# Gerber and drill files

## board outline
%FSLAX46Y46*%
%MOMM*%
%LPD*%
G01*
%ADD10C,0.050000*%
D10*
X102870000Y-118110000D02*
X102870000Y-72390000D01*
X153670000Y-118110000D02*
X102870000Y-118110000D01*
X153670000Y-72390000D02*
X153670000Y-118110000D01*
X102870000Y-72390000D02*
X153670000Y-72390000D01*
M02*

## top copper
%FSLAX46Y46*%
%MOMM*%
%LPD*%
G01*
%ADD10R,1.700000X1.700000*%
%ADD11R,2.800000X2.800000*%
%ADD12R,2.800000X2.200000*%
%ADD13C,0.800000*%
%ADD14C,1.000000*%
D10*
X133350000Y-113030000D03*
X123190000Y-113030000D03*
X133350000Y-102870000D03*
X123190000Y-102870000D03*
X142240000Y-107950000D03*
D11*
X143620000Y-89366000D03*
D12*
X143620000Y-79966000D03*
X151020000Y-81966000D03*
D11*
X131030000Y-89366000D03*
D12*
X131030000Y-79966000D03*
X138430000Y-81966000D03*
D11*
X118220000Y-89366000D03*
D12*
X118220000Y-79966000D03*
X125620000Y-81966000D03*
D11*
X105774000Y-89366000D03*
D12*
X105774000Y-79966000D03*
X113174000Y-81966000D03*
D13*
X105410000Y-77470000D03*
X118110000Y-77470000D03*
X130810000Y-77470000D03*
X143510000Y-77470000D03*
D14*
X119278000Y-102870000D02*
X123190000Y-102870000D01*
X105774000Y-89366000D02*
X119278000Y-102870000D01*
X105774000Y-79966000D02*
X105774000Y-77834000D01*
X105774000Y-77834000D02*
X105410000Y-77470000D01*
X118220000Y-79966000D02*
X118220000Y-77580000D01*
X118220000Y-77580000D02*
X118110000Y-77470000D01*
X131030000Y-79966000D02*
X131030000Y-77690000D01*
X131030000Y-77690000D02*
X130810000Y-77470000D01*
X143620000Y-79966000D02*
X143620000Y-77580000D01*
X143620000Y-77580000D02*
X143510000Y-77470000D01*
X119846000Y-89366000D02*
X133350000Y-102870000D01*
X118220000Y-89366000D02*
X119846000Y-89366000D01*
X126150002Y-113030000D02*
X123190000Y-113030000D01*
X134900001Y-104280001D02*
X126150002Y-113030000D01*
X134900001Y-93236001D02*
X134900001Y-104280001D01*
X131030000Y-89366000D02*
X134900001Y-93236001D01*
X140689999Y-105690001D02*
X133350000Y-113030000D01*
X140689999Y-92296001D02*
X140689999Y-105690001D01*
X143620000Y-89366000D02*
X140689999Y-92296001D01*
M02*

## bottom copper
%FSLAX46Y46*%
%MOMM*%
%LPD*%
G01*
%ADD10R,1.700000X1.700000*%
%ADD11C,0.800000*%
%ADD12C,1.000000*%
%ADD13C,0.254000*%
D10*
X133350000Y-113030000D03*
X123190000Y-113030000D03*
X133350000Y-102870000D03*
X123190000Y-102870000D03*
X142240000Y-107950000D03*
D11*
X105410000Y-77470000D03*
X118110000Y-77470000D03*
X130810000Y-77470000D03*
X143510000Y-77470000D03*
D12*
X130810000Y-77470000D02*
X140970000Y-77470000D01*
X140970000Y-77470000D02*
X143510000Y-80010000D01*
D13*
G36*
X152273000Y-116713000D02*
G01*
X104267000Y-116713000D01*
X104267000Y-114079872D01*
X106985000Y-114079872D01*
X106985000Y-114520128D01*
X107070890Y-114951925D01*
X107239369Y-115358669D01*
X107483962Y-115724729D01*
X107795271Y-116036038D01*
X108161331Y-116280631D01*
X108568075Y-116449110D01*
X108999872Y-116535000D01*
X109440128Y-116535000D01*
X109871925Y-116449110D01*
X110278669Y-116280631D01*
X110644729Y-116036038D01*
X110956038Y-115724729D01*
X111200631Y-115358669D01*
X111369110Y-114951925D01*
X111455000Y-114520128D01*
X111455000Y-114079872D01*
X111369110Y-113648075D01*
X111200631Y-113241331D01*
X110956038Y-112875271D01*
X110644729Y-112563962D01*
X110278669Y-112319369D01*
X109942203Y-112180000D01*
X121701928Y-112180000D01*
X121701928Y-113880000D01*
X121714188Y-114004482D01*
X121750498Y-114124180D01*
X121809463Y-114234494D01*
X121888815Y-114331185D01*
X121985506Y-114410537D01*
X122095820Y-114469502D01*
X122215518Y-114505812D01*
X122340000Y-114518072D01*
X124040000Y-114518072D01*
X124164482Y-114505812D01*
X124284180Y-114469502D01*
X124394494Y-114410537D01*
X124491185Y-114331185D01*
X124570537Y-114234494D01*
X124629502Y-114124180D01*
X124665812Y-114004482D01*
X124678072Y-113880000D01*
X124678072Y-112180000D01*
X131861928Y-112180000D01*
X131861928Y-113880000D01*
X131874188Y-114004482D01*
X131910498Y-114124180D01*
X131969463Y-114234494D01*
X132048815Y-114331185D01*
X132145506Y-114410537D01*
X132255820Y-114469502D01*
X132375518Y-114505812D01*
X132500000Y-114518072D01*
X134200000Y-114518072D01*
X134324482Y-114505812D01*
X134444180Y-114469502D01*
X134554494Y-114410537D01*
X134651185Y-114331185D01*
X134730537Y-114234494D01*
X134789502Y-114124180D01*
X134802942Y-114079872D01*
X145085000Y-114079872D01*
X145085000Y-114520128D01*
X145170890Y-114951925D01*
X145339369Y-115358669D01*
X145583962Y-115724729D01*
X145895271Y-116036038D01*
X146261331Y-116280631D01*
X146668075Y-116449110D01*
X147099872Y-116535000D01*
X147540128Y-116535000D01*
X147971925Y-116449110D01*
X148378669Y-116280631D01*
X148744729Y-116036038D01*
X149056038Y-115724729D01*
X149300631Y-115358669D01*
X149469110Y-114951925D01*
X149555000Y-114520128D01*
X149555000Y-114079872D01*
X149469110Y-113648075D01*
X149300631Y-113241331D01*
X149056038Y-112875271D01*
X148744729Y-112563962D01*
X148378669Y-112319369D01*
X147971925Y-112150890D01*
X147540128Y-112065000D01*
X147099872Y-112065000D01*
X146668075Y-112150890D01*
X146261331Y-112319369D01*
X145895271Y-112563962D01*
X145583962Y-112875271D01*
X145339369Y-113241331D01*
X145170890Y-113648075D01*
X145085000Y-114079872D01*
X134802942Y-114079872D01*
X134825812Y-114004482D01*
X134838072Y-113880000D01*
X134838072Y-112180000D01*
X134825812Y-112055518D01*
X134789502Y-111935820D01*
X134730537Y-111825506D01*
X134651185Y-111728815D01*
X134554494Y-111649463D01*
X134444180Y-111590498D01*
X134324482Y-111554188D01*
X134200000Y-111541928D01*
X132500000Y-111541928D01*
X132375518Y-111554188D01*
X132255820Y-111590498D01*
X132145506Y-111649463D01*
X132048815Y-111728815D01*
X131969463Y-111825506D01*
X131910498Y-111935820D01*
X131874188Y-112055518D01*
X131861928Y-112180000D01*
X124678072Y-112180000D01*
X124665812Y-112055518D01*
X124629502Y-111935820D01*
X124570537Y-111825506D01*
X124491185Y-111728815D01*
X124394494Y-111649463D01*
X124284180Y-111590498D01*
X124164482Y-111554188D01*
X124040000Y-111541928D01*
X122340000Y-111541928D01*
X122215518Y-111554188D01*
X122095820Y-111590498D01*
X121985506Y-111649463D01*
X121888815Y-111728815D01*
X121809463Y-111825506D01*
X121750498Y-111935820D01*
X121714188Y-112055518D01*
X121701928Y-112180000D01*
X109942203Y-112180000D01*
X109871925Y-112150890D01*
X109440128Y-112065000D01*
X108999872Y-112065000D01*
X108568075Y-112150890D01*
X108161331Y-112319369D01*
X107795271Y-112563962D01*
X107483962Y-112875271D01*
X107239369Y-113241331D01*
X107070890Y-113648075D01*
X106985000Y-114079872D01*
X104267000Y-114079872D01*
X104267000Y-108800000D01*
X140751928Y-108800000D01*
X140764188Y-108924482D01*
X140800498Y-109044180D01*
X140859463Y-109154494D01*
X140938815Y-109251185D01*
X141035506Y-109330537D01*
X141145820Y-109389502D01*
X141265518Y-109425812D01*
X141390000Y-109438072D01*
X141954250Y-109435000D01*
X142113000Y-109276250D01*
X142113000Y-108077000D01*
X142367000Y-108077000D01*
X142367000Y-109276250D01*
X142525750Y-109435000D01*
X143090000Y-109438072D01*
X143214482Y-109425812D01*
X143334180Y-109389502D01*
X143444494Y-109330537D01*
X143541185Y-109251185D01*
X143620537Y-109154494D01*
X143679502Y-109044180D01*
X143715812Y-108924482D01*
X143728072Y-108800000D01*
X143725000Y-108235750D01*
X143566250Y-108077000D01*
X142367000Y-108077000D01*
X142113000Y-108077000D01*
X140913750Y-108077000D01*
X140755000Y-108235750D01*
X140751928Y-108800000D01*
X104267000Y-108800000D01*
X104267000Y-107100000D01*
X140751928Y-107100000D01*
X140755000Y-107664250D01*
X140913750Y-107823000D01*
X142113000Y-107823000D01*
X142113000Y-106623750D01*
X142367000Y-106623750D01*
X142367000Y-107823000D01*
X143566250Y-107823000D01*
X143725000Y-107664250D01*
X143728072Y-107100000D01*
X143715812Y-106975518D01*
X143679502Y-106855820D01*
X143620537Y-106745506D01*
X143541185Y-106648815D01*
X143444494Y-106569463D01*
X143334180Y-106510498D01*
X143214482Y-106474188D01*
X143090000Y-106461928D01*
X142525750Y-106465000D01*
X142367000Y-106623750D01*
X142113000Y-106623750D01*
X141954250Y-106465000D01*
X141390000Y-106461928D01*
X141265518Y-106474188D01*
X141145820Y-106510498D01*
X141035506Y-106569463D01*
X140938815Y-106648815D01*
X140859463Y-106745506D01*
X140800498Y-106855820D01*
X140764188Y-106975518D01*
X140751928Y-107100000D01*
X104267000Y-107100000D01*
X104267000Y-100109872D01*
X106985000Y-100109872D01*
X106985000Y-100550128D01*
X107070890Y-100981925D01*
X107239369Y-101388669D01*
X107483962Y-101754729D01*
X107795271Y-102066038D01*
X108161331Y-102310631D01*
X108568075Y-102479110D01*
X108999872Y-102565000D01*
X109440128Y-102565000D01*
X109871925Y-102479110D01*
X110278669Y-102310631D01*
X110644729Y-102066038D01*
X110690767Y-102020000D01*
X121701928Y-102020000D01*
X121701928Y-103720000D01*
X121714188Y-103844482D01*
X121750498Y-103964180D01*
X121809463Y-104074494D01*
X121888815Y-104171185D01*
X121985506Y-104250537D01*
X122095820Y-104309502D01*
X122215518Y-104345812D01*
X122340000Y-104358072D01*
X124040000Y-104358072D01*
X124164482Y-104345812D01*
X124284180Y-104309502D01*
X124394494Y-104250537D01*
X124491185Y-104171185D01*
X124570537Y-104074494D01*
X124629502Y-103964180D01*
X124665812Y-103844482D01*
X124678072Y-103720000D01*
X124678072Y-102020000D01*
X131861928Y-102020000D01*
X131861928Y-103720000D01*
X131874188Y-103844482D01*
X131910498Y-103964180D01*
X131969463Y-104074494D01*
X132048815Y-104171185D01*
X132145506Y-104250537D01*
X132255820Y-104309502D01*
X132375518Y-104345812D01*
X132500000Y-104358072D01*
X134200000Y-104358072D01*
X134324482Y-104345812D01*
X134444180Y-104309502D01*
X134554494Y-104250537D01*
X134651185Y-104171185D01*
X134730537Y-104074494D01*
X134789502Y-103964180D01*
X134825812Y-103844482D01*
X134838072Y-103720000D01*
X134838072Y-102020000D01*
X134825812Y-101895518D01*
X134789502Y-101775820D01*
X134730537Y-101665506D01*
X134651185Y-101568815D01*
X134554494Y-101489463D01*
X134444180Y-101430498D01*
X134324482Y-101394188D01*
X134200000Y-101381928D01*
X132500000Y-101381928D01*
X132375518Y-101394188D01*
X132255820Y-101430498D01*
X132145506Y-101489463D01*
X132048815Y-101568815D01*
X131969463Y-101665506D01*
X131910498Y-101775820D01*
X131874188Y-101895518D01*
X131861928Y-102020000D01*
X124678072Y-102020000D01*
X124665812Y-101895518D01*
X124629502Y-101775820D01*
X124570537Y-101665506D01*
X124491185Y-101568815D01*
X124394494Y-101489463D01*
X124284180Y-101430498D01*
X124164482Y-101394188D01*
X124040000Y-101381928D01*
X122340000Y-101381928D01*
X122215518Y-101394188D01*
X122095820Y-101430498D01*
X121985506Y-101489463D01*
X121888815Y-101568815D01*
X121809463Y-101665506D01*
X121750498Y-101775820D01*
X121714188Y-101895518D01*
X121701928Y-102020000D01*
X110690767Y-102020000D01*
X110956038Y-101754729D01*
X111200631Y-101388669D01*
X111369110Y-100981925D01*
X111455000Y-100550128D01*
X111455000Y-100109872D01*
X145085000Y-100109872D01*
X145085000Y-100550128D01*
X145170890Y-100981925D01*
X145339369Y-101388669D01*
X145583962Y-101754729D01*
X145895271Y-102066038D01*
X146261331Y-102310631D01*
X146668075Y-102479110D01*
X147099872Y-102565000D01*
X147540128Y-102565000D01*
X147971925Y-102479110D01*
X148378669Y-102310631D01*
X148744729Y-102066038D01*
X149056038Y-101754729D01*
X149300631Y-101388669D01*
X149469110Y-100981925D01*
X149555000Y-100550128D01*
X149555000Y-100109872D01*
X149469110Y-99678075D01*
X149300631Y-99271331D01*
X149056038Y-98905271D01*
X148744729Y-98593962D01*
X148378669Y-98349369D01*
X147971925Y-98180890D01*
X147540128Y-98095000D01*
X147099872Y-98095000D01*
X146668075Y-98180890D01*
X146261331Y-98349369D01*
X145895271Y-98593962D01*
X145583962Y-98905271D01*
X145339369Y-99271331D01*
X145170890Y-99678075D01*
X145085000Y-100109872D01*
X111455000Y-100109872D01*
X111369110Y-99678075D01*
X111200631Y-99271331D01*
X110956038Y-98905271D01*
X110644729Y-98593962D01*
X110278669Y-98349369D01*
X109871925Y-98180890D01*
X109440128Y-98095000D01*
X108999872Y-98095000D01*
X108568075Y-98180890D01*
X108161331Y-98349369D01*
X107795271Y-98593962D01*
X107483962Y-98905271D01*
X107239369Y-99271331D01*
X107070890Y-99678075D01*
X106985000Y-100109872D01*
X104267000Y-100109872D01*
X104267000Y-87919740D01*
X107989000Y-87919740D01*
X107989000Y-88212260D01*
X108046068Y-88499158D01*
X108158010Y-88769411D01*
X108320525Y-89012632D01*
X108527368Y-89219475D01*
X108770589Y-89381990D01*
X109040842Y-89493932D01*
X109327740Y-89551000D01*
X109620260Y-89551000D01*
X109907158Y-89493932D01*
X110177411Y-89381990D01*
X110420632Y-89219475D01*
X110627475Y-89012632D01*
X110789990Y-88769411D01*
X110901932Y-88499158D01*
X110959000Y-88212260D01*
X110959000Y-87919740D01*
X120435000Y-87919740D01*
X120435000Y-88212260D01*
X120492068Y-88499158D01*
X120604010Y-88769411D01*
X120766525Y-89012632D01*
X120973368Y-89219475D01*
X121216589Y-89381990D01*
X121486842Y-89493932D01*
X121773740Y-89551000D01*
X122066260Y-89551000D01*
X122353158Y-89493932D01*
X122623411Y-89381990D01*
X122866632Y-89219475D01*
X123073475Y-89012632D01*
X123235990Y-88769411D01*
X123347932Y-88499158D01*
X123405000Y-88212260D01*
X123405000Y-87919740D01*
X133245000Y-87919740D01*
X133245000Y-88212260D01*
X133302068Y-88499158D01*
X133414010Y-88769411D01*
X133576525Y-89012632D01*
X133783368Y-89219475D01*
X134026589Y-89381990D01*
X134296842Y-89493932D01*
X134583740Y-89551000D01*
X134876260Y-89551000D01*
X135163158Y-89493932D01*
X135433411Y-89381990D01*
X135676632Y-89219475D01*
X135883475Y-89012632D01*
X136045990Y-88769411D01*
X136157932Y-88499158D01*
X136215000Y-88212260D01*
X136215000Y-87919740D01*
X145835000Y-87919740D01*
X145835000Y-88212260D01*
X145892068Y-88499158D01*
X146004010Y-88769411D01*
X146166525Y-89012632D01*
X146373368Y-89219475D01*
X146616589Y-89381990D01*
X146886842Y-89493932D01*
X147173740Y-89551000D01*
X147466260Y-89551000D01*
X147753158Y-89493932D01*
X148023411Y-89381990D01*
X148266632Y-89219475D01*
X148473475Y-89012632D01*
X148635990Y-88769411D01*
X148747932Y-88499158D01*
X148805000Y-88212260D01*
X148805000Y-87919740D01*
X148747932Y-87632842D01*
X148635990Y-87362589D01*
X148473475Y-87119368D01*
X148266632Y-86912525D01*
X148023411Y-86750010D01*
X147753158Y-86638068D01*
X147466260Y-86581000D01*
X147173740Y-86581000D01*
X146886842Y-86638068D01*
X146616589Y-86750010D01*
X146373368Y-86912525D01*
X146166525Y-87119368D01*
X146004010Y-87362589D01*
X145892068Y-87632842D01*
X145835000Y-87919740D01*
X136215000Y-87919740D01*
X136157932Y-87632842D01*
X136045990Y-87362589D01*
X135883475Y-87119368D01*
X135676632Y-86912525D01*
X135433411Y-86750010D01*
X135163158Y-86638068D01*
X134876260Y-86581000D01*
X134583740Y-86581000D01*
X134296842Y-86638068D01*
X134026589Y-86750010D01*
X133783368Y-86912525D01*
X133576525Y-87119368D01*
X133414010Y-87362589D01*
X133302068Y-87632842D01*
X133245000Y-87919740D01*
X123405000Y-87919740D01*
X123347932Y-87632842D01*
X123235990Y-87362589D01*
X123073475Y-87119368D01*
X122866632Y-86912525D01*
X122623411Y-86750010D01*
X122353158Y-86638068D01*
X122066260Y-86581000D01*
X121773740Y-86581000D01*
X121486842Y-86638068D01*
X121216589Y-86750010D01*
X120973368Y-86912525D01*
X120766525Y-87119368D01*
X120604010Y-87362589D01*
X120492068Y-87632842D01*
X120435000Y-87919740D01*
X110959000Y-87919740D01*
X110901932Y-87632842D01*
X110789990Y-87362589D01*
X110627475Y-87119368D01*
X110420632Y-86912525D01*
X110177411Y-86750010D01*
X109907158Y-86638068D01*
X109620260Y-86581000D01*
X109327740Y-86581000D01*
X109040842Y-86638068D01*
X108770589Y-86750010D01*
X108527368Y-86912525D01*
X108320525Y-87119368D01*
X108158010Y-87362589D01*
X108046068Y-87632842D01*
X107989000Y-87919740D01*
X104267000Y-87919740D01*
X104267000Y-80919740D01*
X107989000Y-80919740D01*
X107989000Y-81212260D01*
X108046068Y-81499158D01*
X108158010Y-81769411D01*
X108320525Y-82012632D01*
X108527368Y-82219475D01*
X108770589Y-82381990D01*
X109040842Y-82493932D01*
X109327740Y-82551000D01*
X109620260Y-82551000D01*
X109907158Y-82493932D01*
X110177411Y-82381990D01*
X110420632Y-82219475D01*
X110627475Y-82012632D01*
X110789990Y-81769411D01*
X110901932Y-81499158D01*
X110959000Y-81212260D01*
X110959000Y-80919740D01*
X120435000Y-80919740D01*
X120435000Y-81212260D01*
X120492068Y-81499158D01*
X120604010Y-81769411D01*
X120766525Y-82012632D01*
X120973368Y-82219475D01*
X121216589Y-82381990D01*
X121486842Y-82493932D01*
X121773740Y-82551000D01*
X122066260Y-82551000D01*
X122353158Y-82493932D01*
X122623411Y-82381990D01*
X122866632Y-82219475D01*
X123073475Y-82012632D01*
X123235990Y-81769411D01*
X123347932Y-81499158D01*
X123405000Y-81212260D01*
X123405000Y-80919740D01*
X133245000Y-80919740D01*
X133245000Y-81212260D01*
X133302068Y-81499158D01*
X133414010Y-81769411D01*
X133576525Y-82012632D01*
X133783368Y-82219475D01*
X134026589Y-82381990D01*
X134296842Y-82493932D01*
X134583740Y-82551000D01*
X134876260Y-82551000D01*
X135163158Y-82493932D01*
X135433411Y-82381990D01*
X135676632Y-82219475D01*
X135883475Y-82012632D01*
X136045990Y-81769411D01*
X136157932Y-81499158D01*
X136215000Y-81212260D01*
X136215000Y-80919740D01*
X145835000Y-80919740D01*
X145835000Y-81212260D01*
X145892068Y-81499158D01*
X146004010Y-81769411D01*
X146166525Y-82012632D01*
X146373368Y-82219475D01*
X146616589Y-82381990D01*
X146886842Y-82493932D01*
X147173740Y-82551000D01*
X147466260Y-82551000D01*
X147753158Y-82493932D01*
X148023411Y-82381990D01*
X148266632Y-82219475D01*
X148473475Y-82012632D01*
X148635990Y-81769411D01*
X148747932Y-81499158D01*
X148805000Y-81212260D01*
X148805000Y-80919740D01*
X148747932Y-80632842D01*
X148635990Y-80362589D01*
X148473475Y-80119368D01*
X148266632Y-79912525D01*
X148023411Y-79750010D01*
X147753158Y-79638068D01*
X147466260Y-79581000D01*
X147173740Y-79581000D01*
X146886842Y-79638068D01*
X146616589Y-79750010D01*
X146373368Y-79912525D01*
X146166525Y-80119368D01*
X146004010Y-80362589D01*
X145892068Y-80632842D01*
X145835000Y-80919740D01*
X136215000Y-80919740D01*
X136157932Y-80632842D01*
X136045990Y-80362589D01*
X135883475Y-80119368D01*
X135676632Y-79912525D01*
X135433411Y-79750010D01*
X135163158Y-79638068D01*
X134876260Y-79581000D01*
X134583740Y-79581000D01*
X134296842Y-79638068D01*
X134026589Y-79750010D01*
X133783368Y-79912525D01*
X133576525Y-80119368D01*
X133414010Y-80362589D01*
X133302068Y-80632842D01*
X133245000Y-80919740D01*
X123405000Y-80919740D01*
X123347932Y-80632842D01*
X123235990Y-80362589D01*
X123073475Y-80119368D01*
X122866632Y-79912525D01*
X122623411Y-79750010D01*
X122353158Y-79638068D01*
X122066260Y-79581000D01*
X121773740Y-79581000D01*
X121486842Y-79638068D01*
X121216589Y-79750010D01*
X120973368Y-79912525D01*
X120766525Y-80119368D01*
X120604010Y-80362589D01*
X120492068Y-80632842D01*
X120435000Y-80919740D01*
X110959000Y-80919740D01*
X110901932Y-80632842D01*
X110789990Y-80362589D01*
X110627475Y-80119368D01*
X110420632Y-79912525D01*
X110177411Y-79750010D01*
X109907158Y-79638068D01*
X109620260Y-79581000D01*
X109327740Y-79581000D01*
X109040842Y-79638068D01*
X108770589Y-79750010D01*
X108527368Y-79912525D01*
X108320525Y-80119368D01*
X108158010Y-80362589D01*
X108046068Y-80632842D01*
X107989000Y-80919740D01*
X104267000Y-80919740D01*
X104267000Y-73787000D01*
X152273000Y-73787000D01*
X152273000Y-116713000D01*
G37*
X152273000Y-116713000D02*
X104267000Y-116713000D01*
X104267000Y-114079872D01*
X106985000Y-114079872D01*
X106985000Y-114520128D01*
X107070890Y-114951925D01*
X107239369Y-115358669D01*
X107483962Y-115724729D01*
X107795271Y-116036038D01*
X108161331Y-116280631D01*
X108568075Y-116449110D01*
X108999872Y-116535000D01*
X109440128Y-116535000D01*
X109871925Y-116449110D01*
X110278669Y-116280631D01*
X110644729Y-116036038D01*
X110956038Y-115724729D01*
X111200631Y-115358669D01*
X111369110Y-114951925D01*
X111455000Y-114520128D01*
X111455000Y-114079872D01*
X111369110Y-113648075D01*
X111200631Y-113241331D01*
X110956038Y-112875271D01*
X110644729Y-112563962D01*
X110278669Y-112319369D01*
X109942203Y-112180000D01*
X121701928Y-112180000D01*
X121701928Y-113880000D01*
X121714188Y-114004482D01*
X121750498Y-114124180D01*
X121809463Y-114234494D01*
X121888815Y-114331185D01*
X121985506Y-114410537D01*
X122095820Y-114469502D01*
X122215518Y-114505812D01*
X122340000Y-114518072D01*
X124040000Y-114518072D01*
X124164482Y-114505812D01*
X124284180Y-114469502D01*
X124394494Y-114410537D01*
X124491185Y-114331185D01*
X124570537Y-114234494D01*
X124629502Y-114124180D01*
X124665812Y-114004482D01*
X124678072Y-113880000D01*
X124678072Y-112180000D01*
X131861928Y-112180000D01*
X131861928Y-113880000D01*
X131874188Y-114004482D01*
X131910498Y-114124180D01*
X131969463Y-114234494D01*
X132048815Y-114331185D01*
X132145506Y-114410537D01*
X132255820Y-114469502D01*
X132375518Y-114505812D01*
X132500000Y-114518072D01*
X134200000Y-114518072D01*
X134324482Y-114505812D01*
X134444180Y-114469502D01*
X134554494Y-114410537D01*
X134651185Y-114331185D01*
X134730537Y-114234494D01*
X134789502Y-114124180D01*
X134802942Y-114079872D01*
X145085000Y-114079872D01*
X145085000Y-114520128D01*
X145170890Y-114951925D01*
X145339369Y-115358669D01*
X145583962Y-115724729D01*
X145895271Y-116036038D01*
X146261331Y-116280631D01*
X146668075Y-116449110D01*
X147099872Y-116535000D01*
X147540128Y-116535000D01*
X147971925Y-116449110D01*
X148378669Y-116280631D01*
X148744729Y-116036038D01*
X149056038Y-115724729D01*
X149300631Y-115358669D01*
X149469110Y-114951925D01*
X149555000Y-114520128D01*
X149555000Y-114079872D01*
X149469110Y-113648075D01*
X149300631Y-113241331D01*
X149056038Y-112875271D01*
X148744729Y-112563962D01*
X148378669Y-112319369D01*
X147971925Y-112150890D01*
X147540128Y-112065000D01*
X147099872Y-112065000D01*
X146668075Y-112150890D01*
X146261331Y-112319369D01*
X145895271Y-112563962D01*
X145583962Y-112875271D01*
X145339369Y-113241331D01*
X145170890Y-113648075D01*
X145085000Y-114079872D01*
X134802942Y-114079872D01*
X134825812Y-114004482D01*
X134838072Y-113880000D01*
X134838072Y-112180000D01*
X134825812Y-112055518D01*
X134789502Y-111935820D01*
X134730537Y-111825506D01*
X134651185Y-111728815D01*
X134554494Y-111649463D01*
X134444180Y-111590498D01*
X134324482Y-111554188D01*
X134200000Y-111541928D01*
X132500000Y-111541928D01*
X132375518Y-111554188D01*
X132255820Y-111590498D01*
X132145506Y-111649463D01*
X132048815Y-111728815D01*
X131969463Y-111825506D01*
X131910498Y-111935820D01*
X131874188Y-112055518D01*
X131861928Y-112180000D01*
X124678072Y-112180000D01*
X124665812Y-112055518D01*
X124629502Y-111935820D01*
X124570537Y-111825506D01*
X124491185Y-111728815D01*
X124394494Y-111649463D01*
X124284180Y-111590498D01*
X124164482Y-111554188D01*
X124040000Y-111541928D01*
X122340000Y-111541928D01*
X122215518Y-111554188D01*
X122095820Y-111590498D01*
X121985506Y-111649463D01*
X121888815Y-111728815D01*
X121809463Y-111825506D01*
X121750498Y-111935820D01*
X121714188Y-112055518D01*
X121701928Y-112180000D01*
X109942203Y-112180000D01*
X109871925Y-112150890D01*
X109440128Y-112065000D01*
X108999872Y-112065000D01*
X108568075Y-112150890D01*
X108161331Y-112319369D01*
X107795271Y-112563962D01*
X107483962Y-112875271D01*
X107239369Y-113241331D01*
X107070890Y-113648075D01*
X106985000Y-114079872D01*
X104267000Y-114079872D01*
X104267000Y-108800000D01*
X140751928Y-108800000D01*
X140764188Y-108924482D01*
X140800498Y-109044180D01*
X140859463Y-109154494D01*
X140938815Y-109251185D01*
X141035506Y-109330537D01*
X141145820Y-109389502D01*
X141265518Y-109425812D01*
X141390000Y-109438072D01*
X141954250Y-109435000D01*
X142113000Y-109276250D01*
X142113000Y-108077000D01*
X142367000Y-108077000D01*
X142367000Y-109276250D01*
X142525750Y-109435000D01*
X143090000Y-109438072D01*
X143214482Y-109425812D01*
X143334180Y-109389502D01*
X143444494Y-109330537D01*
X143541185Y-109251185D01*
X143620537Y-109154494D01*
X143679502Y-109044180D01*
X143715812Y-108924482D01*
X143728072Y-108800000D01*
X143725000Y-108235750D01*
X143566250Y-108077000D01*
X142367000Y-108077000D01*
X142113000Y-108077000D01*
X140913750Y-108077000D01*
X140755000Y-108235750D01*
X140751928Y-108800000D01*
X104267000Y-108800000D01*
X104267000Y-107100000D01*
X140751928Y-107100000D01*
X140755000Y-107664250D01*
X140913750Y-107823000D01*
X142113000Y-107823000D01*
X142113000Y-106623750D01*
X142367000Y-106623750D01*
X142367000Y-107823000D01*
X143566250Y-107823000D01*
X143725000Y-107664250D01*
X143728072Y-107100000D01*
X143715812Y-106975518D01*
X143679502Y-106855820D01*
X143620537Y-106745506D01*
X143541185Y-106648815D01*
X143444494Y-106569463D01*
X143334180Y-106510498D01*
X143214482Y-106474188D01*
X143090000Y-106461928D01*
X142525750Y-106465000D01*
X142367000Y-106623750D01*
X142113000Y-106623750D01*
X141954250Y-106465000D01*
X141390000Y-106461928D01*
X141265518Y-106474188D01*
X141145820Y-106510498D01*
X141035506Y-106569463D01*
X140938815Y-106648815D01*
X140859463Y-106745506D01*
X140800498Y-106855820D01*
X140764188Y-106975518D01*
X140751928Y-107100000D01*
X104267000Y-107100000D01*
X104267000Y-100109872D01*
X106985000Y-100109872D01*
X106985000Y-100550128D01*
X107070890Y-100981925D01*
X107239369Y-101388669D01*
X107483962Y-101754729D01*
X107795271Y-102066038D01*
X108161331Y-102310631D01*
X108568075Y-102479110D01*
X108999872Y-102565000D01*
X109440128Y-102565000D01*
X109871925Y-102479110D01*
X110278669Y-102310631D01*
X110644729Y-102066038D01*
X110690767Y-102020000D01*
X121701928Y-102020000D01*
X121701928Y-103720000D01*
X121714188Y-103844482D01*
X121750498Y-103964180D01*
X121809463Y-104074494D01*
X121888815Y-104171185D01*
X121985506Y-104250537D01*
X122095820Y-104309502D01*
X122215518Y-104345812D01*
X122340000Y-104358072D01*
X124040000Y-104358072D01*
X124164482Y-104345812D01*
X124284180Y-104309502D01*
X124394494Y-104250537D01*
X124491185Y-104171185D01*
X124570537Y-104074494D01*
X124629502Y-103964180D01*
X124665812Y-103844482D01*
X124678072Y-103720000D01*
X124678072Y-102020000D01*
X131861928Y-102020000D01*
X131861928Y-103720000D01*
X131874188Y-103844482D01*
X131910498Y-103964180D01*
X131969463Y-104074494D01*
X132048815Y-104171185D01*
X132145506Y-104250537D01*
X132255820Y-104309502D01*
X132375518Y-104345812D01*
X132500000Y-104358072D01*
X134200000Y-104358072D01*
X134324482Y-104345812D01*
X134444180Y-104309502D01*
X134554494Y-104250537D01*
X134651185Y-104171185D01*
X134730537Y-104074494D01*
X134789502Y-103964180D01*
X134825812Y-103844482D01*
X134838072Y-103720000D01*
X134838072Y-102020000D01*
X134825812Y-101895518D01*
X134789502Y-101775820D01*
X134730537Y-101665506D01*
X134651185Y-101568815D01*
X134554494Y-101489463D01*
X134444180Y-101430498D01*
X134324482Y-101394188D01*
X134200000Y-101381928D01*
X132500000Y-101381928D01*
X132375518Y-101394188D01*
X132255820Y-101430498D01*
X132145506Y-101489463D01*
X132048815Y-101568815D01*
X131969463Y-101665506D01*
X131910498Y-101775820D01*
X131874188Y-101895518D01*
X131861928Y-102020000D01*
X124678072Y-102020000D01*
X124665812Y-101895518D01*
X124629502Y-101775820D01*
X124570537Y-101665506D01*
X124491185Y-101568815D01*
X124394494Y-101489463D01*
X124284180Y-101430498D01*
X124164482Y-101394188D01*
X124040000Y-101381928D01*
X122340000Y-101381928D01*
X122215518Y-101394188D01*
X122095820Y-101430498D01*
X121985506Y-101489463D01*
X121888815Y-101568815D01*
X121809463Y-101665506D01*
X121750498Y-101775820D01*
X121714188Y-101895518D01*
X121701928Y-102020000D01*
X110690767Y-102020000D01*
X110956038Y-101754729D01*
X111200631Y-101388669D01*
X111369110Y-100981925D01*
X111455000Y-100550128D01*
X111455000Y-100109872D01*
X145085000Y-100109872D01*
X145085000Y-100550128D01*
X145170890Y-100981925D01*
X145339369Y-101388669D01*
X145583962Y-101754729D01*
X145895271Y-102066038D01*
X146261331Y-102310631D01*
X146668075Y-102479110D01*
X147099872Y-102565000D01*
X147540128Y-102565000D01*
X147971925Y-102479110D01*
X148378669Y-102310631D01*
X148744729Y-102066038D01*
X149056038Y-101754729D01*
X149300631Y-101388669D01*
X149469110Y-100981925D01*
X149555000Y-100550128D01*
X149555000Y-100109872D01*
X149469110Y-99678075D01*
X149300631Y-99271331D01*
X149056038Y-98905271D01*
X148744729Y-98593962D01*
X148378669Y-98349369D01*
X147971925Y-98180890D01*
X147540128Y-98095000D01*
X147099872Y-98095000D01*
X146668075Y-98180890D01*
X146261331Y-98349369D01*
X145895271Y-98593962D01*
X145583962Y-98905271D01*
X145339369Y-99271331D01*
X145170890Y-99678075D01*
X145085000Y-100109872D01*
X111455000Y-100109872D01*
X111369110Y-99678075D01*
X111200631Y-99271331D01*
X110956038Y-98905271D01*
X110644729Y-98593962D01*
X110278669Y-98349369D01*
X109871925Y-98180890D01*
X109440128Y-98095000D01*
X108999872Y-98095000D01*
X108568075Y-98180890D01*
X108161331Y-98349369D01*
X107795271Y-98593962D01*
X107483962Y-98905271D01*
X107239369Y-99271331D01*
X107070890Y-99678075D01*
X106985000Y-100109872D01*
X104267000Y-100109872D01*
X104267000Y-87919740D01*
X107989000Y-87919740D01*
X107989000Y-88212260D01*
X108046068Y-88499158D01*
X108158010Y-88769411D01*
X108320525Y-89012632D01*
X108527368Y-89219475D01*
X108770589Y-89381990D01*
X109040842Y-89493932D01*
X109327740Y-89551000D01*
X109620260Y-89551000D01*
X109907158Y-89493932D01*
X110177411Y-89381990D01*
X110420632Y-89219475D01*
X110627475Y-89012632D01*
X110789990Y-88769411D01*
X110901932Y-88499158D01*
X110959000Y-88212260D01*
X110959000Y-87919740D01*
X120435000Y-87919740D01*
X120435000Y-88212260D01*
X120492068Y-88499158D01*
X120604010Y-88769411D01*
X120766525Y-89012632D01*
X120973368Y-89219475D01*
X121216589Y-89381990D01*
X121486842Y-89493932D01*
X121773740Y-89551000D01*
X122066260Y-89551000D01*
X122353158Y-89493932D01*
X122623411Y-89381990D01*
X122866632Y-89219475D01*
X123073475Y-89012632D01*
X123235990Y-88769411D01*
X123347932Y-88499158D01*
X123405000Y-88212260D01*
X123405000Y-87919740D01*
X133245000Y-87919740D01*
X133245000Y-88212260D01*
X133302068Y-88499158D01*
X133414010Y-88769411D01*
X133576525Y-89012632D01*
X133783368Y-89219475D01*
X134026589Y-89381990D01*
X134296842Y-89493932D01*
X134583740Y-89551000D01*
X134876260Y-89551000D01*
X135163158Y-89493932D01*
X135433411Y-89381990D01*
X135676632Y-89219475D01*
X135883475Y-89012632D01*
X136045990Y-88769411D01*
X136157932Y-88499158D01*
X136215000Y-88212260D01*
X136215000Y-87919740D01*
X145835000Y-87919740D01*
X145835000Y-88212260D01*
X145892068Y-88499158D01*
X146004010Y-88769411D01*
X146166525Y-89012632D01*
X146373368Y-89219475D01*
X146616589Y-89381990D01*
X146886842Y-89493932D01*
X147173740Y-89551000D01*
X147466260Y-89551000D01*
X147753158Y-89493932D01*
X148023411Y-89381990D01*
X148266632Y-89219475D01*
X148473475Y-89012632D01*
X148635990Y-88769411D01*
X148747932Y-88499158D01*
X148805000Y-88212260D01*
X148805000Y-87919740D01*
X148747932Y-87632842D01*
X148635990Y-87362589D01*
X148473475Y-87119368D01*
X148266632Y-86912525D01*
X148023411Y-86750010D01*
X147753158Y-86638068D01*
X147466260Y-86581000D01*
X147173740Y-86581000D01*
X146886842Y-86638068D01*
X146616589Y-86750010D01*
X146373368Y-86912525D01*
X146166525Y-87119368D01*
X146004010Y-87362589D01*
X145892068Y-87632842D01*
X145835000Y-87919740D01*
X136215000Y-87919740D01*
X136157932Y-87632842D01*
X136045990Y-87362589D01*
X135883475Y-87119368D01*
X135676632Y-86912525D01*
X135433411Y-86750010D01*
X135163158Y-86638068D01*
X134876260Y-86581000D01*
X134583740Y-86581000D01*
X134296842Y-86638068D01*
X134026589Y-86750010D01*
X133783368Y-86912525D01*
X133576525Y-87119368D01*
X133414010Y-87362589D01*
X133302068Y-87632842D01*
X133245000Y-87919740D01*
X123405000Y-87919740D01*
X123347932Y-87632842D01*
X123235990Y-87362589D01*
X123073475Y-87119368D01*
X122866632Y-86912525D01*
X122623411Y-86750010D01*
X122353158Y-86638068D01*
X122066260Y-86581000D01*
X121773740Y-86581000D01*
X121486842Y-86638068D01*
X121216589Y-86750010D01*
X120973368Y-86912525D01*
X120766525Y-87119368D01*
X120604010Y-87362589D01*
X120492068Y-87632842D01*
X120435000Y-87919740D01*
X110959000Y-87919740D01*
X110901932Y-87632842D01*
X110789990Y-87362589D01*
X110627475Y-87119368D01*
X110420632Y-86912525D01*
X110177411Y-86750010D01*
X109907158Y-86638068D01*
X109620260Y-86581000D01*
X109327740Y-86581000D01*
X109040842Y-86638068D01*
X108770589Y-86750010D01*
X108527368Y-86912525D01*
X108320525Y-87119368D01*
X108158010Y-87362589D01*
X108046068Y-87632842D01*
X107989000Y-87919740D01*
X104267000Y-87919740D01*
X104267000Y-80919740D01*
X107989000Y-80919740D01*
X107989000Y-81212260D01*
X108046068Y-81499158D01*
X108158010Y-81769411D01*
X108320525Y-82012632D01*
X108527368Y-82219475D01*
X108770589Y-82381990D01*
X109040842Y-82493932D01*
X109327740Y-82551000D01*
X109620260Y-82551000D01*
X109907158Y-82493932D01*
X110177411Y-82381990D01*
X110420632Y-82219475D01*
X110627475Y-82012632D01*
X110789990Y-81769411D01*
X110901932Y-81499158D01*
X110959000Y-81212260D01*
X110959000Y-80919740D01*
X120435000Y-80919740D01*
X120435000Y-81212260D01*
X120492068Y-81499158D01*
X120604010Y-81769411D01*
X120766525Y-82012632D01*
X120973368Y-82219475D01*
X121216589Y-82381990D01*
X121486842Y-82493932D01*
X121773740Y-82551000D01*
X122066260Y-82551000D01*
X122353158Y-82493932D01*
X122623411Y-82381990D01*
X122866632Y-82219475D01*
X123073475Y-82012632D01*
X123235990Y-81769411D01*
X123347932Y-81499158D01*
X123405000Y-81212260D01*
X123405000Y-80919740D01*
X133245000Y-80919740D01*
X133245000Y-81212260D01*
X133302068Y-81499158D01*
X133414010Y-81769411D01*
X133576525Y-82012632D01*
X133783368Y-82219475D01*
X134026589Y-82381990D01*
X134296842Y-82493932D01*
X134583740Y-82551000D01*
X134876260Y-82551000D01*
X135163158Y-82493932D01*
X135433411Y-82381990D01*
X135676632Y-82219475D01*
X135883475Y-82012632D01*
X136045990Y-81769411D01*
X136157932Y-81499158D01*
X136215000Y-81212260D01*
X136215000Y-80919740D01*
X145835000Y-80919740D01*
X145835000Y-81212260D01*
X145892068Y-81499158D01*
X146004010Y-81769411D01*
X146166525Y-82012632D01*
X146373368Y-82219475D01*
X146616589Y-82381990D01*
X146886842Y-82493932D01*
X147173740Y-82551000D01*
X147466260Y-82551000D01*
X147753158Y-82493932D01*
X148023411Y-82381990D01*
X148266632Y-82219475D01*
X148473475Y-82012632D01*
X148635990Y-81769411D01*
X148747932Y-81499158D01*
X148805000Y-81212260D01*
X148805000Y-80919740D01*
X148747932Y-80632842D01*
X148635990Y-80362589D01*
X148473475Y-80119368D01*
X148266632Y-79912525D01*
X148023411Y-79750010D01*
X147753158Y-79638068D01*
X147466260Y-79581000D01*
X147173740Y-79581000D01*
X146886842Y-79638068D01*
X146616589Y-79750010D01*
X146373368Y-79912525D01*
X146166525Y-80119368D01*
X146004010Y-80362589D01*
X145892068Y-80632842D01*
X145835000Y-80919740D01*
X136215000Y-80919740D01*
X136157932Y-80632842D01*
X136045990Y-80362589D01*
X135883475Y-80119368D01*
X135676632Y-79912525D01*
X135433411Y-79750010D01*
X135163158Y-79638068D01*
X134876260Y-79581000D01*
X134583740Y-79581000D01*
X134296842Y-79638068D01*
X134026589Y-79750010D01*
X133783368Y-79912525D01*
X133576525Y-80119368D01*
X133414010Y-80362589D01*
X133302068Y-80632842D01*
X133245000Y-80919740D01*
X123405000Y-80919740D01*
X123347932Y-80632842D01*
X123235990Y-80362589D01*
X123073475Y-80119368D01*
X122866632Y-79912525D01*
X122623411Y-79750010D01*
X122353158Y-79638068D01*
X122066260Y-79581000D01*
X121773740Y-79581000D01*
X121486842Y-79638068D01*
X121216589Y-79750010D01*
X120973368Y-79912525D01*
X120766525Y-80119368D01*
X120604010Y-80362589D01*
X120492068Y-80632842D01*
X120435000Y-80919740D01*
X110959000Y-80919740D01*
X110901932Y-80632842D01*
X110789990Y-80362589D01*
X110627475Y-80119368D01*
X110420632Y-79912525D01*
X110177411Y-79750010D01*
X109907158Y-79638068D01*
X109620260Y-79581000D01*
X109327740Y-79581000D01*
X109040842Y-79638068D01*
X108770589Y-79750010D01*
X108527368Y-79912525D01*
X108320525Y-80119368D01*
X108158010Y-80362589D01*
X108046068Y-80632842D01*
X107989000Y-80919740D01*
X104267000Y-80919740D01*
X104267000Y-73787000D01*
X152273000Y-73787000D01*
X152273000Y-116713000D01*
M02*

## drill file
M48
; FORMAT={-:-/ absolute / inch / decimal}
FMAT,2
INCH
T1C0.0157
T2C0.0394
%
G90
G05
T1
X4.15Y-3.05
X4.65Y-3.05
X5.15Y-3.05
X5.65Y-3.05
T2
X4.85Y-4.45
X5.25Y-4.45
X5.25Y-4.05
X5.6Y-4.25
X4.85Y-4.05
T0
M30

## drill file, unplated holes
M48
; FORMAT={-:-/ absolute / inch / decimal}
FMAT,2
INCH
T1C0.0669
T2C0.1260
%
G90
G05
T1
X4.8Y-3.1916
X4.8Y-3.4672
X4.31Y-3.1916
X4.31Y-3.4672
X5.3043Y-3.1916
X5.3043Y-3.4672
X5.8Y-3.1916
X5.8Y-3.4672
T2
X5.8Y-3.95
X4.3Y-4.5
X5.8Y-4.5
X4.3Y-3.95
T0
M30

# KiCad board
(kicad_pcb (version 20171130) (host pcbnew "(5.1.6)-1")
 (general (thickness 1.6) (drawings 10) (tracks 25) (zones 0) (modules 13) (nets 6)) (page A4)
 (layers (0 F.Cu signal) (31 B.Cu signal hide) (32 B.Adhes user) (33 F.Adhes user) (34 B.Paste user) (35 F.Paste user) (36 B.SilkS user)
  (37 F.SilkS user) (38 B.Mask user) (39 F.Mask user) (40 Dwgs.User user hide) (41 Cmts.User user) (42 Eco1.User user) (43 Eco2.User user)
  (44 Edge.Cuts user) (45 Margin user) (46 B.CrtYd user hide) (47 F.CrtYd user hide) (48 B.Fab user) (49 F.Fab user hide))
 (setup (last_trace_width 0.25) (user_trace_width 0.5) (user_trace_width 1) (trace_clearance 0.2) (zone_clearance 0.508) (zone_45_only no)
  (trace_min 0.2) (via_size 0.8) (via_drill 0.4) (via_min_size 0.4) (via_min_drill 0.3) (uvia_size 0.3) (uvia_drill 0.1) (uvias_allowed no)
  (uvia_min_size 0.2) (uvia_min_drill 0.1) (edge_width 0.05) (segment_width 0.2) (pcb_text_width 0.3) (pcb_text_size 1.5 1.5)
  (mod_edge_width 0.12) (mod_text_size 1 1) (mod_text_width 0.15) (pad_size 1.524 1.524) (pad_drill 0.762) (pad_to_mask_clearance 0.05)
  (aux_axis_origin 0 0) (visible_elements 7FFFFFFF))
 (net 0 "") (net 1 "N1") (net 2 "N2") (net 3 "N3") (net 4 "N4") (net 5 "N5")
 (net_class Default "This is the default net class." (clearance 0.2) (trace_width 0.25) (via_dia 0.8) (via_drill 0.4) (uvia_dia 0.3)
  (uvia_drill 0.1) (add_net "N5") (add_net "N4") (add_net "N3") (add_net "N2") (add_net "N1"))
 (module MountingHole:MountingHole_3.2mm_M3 (layer F.Cu) (at 109.22 114.3)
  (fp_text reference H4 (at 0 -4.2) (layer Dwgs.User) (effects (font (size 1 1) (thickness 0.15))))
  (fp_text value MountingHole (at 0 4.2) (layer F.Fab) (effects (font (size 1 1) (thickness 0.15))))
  (pad 1 np_thru_hole circle (at 0 0) (size 3.2 3.2) (drill 3.2) (layers *.Cu *.Mask)))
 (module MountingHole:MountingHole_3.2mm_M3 (layer F.Cu) (at 109.22 100.33)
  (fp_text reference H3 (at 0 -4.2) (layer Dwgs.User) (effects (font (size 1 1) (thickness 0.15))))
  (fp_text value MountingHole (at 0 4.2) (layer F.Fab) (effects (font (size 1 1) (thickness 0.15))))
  (pad 1 np_thru_hole circle (at 0 0) (size 3.2 3.2) (drill 3.2) (layers *.Cu *.Mask)))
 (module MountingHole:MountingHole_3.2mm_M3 (layer F.Cu) (at 147.32 100.33)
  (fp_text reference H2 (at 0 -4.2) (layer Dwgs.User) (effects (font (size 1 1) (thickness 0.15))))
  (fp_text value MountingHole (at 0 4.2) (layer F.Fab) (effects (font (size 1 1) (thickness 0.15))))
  (pad 1 np_thru_hole circle (at 0 0) (size 3.2 3.2) (drill 3.2) (layers *.Cu *.Mask)))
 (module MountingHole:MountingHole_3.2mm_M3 (layer F.Cu) (at 147.32 114.3)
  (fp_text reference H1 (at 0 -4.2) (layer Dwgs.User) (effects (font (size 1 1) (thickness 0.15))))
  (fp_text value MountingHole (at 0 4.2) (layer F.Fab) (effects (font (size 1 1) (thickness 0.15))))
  (pad 1 np_thru_hole circle (at 0 0) (size 3.2 3.2) (drill 3.2) (layers *.Cu *.Mask)))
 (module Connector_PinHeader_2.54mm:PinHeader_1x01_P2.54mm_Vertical (layer F.Cu) (at 133.35 113.03)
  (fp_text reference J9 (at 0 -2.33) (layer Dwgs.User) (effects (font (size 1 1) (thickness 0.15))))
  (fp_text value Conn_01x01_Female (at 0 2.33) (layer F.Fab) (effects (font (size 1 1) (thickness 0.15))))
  (pad 1 thru_hole rect (at 0 0) (size 1.7 1.7) (drill 1) (layers *.Cu *.Mask) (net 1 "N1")))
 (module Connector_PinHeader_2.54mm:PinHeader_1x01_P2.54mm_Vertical (layer F.Cu) (at 123.19 113.03)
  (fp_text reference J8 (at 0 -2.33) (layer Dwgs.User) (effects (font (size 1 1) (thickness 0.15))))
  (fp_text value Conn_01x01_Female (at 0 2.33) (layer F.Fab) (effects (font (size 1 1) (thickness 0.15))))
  (pad 1 thru_hole rect (at 0 0) (size 1.7 1.7) (drill 1) (layers *.Cu *.Mask) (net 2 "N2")))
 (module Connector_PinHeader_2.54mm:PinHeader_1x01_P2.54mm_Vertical (layer F.Cu) (at 133.35 102.87)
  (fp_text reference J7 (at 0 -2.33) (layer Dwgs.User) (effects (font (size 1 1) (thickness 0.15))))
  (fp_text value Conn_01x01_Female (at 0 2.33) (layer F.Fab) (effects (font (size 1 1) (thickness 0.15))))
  (pad 1 thru_hole rect (at 0 0) (size 1.7 1.7) (drill 1) (layers *.Cu *.Mask) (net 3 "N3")))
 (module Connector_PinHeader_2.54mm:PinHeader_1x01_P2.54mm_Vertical (layer F.Cu) (at 123.19 102.87)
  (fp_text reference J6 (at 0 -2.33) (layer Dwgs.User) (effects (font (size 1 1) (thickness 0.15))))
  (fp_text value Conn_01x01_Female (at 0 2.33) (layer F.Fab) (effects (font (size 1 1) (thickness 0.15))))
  (pad 1 thru_hole rect (at 0 0) (size 1.7 1.7) (drill 1) (layers *.Cu *.Mask) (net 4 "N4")))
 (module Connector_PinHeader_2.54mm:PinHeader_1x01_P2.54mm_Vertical (layer F.Cu) (at 142.24 107.95)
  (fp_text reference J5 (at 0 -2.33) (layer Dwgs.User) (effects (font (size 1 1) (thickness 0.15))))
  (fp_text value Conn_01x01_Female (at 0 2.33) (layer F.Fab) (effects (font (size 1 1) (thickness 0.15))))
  (pad 1 thru_hole rect (at 0 0) (size 1.7 1.7) (drill 1) (layers *.Cu *.Mask) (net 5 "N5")))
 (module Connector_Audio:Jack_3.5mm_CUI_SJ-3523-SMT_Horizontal (layer F.Cu) (at 147.32 83.566)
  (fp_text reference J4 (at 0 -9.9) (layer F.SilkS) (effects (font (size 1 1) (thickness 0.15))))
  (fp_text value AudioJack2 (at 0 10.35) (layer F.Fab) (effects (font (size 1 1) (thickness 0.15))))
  (pad "" np_thru_hole circle (at 0 4.5) (size 1.7 1.7) (drill 1.7) (layers *.Cu *.Mask))
  (pad "" np_thru_hole circle (at 0 -2.5) (size 1.7 1.7) (drill 1.7) (layers *.Cu *.Mask))
  (pad T smd rect (at -3.7 5.8) (size 2.8 2.8) (layers F.Cu F.Paste F.Mask) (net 1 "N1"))
  (pad S smd rect (at -3.7 -3.6) (size 2.8 2.2) (layers F.Cu F.Paste F.Mask) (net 5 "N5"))
  (pad R smd rect (at 3.7 -1.6) (size 2.8 2.2) (layers F.Cu F.Paste F.Mask)))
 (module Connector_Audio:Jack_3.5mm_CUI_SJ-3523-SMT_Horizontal (layer F.Cu) (at 134.73 83.566)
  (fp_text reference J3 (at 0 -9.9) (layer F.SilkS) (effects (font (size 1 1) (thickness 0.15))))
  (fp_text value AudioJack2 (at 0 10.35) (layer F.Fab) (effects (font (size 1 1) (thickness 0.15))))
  (pad "" np_thru_hole circle (at 0 4.5) (size 1.7 1.7) (drill 1.7) (layers *.Cu *.Mask))
  (pad "" np_thru_hole circle (at 0 -2.5) (size 1.7 1.7) (drill 1.7) (layers *.Cu *.Mask))
  (pad T smd rect (at -3.7 5.8) (size 2.8 2.8) (layers F.Cu F.Paste F.Mask) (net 2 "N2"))
  (pad S smd rect (at -3.7 -3.6) (size 2.8 2.2) (layers F.Cu F.Paste F.Mask) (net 5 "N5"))
  (pad R smd rect (at 3.7 -1.6) (size 2.8 2.2) (layers F.Cu F.Paste F.Mask)))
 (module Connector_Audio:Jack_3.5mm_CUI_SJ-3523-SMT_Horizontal (layer F.Cu) (at 121.92 83.566)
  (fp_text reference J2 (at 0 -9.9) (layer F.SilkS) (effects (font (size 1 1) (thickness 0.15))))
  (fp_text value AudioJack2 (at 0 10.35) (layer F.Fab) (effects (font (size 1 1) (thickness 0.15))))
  (pad "" np_thru_hole circle (at 0 4.5) (size 1.7 1.7) (drill 1.7) (layers *.Cu *.Mask))
  (pad "" np_thru_hole circle (at 0 -2.5) (size 1.7 1.7) (drill 1.7) (layers *.Cu *.Mask))
  (pad T smd rect (at -3.7 5.8) (size 2.8 2.8) (layers F.Cu F.Paste F.Mask) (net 3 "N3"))
  (pad S smd rect (at -3.7 -3.6) (size 2.8 2.2) (layers F.Cu F.Paste F.Mask) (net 5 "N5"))
  (pad R smd rect (at 3.7 -1.6) (size 2.8 2.2) (layers F.Cu F.Paste F.Mask)))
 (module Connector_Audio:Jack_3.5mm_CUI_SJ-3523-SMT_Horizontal (layer F.Cu) (at 109.474 83.566)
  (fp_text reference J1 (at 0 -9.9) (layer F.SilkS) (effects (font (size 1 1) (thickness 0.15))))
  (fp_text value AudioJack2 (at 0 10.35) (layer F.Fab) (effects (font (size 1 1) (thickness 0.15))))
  (pad "" np_thru_hole circle (at 0 4.5) (size 1.7 1.7) (drill 1.7) (layers *.Cu *.Mask))
  (pad "" np_thru_hole circle (at 0 -2.5) (size 1.7 1.7) (drill 1.7) (layers *.Cu *.Mask))
  (pad T smd rect (at -3.7 5.8) (size 2.8 2.8) (layers F.Cu F.Paste F.Mask) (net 4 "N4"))
  (pad S smd rect (at -3.7 -3.6) (size 2.8 2.2) (layers F.Cu F.Paste F.Mask) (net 5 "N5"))
  (pad R smd rect (at 3.7 -1.6) (size 2.8 2.2) (layers F.Cu F.Paste F.Mask)))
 (gr_line (start 102.87 118.11) (end 102.87 72.39) (layer Edge.Cuts) (width 0.05))
 (gr_line (start 153.67 118.11) (end 102.87 118.11) (layer Edge.Cuts) (width 0.05))
 (gr_line (start 153.67 72.39) (end 153.67 118.11) (layer Edge.Cuts) (width 0.05))
 (gr_line (start 102.87 72.39) (end 153.67 72.39) (layer Edge.Cuts) (width 0.05))
 (segment (start 119.278 102.87) (end 123.19 102.87) (width 1) (layer F.Cu) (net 4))
 (segment (start 105.774 89.366) (end 119.278 102.87) (width 1) (layer F.Cu) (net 4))
 (segment (start 105.774 79.966) (end 105.774 77.834) (width 1) (layer F.Cu) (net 5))
 (via (at 105.41 77.47) (size 0.8) (drill 0.4) (layers F.Cu B.Cu) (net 5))
 (segment (start 105.774 77.834) (end 105.41 77.47) (width 1) (layer F.Cu) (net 5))
 (via (at 118.11 77.47) (size 0.8) (drill 0.4) (layers F.Cu B.Cu) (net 5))
 (segment (start 118.22 79.966) (end 118.22 77.58) (width 1) (layer F.Cu) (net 5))
 (segment (start 118.22 77.58) (end 118.11 77.47) (width 1) (layer F.Cu) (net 5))
 (segment (start 131.03 79.966) (end 131.03 77.69) (width 1) (layer F.Cu) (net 5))
 (via (at 130.81 77.47) (size 0.8) (drill 0.4) (layers F.Cu B.Cu) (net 5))
 (segment (start 131.03 77.69) (end 130.81 77.47) (width 1) (layer F.Cu) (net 5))
 (segment (start 130.81 77.47) (end 140.97 77.47) (width 1) (layer B.Cu) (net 5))
 (segment (start 140.97 77.47) (end 143.51 80.01) (width 1) (layer B.Cu) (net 5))
 (via (at 143.51 77.47) (size 0.8) (drill 0.4) (layers F.Cu B.Cu) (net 5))
 (segment (start 143.62 79.966) (end 143.62 77.58) (width 1) (layer F.Cu) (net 5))
 (segment (start 143.62 77.58) (end 143.51 77.47) (width 1) (layer F.Cu) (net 5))
 (segment (start 119.846 89.366) (end 133.35 102.87) (width 1) (layer F.Cu) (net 3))
 (segment (start 118.22 89.366) (end 119.846 89.366) (width 1) (layer F.Cu) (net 3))
 (segment (start 126.150002 113.03) (end 123.19 113.03) (width 1) (layer F.Cu) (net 2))
 (segment (start 134.900001 104.280001) (end 126.150002 113.03) (width 1) (layer F.Cu) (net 2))
 (segment (start 134.900001 93.236001) (end 134.900001 104.280001) (width 1) (layer F.Cu) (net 2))
 (segment (start 131.03 89.366) (end 134.900001 93.236001) (width 1) (layer F.Cu) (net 2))
 (segment (start 140.689999 105.690001) (end 133.35 113.03) (width 1) (layer F.Cu) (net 1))
 (segment (start 140.689999 92.296001) (end 140.689999 105.690001) (width 1) (layer F.Cu) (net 1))
 (segment (start 143.62 89.366) (end 140.689999 92.296001) (width 1) (layer F.Cu) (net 1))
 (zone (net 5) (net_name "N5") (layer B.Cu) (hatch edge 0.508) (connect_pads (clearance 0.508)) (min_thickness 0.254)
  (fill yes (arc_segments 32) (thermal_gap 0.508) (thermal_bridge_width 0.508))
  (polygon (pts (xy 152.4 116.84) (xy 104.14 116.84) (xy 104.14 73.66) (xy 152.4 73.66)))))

